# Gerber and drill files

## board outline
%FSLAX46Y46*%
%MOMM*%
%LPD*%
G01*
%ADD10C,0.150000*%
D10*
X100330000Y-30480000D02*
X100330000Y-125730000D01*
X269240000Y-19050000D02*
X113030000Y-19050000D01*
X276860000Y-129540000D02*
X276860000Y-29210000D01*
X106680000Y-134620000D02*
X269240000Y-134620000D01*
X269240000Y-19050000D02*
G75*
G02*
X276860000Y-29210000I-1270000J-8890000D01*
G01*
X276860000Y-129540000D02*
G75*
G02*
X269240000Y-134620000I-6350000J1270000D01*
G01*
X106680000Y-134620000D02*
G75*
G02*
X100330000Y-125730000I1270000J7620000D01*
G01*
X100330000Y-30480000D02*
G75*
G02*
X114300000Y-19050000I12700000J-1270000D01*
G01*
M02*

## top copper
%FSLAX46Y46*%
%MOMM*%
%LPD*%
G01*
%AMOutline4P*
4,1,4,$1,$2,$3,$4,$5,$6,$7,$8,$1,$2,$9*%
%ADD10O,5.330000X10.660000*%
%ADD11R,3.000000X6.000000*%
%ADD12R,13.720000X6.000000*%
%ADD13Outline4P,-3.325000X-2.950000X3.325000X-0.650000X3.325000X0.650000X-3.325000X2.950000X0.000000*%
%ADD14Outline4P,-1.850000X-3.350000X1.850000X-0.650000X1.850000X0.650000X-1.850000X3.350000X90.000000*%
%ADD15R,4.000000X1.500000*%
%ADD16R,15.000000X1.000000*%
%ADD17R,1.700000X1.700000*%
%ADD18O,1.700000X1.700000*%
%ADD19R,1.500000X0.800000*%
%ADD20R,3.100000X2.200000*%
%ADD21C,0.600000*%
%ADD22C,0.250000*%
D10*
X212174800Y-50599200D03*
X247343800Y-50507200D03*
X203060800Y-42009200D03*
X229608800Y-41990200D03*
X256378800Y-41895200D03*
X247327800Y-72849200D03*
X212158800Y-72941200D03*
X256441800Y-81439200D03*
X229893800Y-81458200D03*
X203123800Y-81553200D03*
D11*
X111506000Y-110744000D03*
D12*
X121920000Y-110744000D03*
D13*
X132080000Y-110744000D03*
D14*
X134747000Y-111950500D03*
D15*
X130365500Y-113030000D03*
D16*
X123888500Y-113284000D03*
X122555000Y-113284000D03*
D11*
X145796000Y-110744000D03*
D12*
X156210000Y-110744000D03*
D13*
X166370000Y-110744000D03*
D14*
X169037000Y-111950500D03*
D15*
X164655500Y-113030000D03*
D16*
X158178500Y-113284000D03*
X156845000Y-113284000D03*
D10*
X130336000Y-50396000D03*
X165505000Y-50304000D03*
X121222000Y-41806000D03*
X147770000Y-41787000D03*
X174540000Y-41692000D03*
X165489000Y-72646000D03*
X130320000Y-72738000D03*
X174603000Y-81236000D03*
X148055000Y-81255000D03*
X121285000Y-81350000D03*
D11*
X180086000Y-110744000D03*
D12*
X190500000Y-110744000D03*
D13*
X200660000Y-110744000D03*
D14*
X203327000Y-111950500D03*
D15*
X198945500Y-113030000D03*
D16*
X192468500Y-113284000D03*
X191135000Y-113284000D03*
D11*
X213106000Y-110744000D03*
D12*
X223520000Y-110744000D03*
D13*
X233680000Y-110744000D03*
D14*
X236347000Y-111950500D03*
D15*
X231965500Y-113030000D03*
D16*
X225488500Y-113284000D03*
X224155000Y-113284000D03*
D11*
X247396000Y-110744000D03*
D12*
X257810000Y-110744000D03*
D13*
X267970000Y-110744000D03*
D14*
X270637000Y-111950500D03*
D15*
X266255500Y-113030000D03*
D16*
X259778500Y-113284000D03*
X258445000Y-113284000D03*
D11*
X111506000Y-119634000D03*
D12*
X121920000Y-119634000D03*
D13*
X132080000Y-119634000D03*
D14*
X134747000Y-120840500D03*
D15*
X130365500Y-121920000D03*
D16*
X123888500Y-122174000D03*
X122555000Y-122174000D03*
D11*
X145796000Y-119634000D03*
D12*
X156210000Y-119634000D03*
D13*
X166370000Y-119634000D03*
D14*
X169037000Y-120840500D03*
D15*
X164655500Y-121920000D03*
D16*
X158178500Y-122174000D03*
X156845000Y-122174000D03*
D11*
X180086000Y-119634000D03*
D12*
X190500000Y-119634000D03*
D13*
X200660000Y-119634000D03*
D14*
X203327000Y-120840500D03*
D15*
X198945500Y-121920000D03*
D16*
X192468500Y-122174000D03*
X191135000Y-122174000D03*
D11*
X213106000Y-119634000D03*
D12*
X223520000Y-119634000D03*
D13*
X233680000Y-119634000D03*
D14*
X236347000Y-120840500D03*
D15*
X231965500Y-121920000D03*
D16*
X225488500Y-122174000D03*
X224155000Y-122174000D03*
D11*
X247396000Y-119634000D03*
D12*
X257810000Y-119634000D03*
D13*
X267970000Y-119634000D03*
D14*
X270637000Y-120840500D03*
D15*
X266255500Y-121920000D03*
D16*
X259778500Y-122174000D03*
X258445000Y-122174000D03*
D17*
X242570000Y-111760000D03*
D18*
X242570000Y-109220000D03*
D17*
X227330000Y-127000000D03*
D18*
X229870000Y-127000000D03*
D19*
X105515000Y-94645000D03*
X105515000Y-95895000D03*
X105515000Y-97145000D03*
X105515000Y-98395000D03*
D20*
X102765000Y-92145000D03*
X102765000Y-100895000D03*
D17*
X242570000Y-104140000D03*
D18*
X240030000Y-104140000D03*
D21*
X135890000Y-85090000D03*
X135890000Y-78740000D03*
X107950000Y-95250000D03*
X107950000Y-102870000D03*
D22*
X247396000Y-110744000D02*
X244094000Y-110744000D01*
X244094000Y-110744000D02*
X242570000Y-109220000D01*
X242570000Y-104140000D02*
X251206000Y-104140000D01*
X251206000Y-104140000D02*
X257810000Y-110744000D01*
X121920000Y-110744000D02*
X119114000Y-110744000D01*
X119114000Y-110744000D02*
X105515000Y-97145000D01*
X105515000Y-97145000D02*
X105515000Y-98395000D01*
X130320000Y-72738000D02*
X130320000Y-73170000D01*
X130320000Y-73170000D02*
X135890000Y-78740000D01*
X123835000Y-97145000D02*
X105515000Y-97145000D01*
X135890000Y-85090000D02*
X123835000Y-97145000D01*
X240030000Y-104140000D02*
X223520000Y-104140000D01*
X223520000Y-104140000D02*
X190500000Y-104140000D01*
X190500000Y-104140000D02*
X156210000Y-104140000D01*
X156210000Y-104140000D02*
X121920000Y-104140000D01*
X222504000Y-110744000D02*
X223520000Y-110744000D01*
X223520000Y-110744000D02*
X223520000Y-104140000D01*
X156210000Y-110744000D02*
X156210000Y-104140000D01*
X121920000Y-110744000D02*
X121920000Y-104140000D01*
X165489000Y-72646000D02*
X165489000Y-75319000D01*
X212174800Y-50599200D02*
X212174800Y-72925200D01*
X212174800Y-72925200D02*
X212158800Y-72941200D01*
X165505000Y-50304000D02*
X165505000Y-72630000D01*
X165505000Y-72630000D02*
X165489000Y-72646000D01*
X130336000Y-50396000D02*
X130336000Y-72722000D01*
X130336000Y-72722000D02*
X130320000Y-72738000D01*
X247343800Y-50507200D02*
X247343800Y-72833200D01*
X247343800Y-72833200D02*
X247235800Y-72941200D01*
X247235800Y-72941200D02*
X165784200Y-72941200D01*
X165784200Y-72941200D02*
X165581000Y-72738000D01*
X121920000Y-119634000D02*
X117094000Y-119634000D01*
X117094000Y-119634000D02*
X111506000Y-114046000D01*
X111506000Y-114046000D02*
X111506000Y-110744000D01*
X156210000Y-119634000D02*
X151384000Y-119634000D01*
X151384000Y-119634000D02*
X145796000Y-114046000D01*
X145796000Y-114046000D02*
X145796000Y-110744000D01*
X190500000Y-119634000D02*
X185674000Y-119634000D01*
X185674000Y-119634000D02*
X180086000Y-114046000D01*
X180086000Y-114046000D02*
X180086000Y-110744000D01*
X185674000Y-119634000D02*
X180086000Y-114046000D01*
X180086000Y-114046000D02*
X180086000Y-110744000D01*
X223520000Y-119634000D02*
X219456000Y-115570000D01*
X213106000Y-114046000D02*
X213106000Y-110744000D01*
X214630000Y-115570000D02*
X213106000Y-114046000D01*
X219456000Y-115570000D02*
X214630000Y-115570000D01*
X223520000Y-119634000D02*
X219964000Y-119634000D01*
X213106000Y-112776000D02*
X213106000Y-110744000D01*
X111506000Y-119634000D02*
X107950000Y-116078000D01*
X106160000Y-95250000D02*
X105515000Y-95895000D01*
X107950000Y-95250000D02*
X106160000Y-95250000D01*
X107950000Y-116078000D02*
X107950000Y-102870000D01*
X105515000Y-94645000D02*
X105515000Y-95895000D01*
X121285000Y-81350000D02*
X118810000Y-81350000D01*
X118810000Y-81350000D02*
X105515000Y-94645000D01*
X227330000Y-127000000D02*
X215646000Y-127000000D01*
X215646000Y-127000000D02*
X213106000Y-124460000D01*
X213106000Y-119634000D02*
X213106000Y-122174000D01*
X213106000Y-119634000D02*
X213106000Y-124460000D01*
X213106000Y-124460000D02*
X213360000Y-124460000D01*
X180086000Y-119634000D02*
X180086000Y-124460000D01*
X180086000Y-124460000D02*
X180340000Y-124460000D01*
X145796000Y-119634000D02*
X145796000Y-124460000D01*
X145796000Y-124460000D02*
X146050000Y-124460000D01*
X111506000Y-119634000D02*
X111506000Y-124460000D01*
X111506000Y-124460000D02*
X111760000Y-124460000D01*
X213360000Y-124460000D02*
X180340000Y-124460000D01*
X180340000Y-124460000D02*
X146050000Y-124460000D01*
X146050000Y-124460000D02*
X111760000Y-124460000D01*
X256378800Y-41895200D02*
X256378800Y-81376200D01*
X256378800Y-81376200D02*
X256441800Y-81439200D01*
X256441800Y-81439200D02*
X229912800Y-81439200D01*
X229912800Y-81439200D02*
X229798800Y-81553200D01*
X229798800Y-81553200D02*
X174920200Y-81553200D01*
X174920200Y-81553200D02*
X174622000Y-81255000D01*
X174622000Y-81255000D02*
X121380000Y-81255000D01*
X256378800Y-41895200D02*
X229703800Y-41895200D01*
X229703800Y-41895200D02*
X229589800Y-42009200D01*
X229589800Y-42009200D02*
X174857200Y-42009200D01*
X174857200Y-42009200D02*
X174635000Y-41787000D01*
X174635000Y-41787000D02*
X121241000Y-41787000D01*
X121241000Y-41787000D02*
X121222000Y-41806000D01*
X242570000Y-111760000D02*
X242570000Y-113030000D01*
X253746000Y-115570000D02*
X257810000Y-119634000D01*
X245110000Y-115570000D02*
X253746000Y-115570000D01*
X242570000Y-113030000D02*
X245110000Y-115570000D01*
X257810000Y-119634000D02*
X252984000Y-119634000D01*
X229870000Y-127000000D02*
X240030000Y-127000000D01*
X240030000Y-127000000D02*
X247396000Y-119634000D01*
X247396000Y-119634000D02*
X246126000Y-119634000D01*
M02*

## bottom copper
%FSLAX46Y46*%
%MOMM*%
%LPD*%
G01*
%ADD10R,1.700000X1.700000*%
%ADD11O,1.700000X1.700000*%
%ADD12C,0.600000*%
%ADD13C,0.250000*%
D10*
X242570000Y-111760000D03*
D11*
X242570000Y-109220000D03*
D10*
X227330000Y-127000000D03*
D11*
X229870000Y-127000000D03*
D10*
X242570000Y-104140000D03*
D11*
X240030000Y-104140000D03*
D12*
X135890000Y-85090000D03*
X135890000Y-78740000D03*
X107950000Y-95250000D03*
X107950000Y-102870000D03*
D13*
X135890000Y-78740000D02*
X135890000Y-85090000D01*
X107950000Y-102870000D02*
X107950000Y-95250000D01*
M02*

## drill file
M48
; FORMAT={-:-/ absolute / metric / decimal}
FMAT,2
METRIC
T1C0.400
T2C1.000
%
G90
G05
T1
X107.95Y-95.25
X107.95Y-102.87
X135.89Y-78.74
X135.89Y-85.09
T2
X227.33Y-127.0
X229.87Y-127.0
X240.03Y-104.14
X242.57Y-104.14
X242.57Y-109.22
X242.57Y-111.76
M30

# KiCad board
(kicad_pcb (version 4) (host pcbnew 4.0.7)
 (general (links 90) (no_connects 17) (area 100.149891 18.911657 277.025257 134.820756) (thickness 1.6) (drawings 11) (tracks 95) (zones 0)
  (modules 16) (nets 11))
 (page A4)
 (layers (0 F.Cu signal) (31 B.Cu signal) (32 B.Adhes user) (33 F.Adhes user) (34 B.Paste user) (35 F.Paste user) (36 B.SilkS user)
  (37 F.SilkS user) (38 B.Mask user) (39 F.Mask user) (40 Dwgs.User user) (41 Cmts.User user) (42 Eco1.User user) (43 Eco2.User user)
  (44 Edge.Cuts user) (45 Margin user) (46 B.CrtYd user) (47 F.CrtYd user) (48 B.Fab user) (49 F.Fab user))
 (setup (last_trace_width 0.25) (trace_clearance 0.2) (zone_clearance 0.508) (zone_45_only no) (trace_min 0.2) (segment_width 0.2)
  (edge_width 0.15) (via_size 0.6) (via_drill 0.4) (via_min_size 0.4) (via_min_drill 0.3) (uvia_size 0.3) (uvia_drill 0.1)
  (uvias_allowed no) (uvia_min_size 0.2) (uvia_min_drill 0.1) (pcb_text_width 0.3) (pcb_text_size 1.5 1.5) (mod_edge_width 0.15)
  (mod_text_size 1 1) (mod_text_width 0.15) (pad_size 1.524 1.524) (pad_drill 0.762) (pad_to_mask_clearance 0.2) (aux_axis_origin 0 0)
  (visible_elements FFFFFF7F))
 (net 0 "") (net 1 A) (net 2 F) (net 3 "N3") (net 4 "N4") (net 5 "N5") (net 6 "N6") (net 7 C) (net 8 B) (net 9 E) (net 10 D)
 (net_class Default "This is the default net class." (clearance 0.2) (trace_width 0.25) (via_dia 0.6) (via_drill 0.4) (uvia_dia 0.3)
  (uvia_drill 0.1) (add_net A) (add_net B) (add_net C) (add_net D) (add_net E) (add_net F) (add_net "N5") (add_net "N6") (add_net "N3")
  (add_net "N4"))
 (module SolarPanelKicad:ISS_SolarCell (layer F.Cu) (at 189.7888 101.8032)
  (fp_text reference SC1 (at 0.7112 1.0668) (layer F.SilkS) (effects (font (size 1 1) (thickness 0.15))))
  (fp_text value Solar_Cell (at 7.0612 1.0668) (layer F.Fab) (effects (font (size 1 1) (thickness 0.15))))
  (pad 1 smd oval (at 22.386 -51.204 180) (size 5.33 10.66) (layers F.Cu F.Paste F.Mask) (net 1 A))
  (pad 1 smd oval (at 57.555 -51.296 180) (size 5.33 10.66) (layers F.Cu F.Paste F.Mask) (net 1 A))
  (pad 2 smd oval (at 13.272 -59.794 180) (size 5.33 10.66) (layers F.Cu F.Paste F.Mask) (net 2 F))
  (pad 2 smd oval (at 39.82 -59.813 180) (size 5.33 10.66) (layers F.Cu F.Paste F.Mask) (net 2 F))
  (pad 2 smd oval (at 66.59 -59.908 180) (size 5.33 10.66) (layers F.Cu F.Paste F.Mask) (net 2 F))
  (pad 1 smd oval (at 57.539 -28.954) (size 5.33 10.66) (layers F.Cu F.Paste F.Mask) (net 1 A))
  (pad 1 smd oval (at 22.37 -28.862) (size 5.33 10.66) (layers F.Cu F.Paste F.Mask) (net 1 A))
  (pad 2 smd oval (at 66.653 -20.364) (size 5.33 10.66) (layers F.Cu F.Paste F.Mask) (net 2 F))
  (pad 2 smd oval (at 40.105 -20.345) (size 5.33 10.66) (layers F.Cu F.Paste F.Mask) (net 2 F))
  (pad 2 smd oval (at 13.335 -20.25) (size 5.33 10.66) (layers F.Cu F.Paste F.Mask) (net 2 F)))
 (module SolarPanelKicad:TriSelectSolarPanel (layer F.Cu) (at 113.03 114.3)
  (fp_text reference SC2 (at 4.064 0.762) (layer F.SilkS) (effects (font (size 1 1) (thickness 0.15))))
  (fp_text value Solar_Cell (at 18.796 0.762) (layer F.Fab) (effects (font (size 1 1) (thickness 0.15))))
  (pad 2 smd rect (at -1.524 -3.556) (size 3 6) (layers F.Cu F.Paste F.Mask) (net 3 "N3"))
  (pad 1 smd rect (at 8.89 -3.556) (size 13.72 6) (layers F.Cu F.Paste F.Mask) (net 1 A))
  (pad 1 smd trapezoid (at 19.05 -3.556) (size 6.65 3.6) (rect_delta 2.3 0) (layers F.Cu F.Paste F.Mask) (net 1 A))
  (pad 1 smd trapezoid (at 21.717 -2.3495 90) (size 3.7 4) (rect_delta 2.7 0) (layers F.Cu F.Paste F.Mask) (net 1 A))
  (pad 1 smd rect (at 17.3355 -1.27) (size 4 1.5) (layers F.Cu F.Paste F.Mask) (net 1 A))
  (pad 1 smd rect (at 10.8585 -1.016) (size 15 1) (layers F.Cu F.Paste F.Mask) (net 1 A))
  (pad 1 smd rect (at 9.525 -1.016) (size 15 1) (layers F.Cu F.Paste F.Mask) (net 1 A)))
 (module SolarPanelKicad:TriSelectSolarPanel (layer F.Cu) (at 147.32 114.3)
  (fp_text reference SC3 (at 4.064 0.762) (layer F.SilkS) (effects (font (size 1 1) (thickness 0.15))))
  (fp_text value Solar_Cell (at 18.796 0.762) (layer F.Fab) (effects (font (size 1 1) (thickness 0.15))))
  (pad 2 smd rect (at -1.524 -3.556) (size 3 6) (layers F.Cu F.Paste F.Mask) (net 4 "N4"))
  (pad 1 smd rect (at 8.89 -3.556) (size 13.72 6) (layers F.Cu F.Paste F.Mask) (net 1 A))
  (pad 1 smd trapezoid (at 19.05 -3.556) (size 6.65 3.6) (rect_delta 2.3 0) (layers F.Cu F.Paste F.Mask) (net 1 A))
  (pad 1 smd trapezoid (at 21.717 -2.3495 90) (size 3.7 4) (rect_delta 2.7 0) (layers F.Cu F.Paste F.Mask) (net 1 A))
  (pad 1 smd rect (at 17.3355 -1.27) (size 4 1.5) (layers F.Cu F.Paste F.Mask) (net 1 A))
  (pad 1 smd rect (at 10.8585 -1.016) (size 15 1) (layers F.Cu F.Paste F.Mask) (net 1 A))
  (pad 1 smd rect (at 9.525 -1.016) (size 15 1) (layers F.Cu F.Paste F.Mask) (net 1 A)))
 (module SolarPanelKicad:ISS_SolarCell (layer F.Cu) (at 107.95 101.6)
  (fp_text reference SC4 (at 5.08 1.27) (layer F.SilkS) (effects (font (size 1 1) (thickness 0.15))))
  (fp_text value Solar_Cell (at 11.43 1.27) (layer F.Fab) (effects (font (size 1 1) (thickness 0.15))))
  (pad 1 smd oval (at 22.386 -51.204 180) (size 5.33 10.66) (layers F.Cu F.Paste F.Mask) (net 1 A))
  (pad 1 smd oval (at 57.555 -51.296 180) (size 5.33 10.66) (layers F.Cu F.Paste F.Mask) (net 1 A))
  (pad 2 smd oval (at 13.272 -59.794 180) (size 5.33 10.66) (layers F.Cu F.Paste F.Mask) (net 2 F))
  (pad 2 smd oval (at 39.82 -59.813 180) (size 5.33 10.66) (layers F.Cu F.Paste F.Mask) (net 2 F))
  (pad 2 smd oval (at 66.59 -59.908 180) (size 5.33 10.66) (layers F.Cu F.Paste F.Mask) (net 2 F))
  (pad 1 smd oval (at 57.539 -28.954) (size 5.33 10.66) (layers F.Cu F.Paste F.Mask) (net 1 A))
  (pad 1 smd oval (at 22.37 -28.862) (size 5.33 10.66) (layers F.Cu F.Paste F.Mask) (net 1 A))
  (pad 2 smd oval (at 66.653 -20.364) (size 5.33 10.66) (layers F.Cu F.Paste F.Mask) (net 2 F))
  (pad 2 smd oval (at 40.105 -20.345) (size 5.33 10.66) (layers F.Cu F.Paste F.Mask) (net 2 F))
  (pad 2 smd oval (at 13.335 -20.25) (size 5.33 10.66) (layers F.Cu F.Paste F.Mask) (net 2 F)))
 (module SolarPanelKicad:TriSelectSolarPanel (layer F.Cu) (at 181.61 114.3)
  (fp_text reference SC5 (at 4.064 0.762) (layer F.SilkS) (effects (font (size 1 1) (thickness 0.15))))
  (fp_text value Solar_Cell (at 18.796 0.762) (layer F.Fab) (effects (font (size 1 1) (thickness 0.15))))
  (pad 2 smd rect (at -1.524 -3.556) (size 3 6) (layers F.Cu F.Paste F.Mask) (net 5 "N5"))
  (pad 1 smd rect (at 8.89 -3.556) (size 13.72 6) (layers F.Cu F.Paste F.Mask) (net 1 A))
  (pad 1 smd trapezoid (at 19.05 -3.556) (size 6.65 3.6) (rect_delta 2.3 0) (layers F.Cu F.Paste F.Mask) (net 1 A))
  (pad 1 smd trapezoid (at 21.717 -2.3495 90) (size 3.7 4) (rect_delta 2.7 0) (layers F.Cu F.Paste F.Mask) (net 1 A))
  (pad 1 smd rect (at 17.3355 -1.27) (size 4 1.5) (layers F.Cu F.Paste F.Mask) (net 1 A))
  (pad 1 smd rect (at 10.8585 -1.016) (size 15 1) (layers F.Cu F.Paste F.Mask) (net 1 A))
  (pad 1 smd rect (at 9.525 -1.016) (size 15 1) (layers F.Cu F.Paste F.Mask) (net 1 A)))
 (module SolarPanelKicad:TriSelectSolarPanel (layer F.Cu) (at 214.63 114.3)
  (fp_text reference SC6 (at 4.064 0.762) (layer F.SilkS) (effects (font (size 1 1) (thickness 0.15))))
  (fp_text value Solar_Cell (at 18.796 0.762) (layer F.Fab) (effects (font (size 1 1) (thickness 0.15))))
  (pad 2 smd rect (at -1.524 -3.556) (size 3 6) (layers F.Cu F.Paste F.Mask) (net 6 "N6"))
  (pad 1 smd rect (at 8.89 -3.556) (size 13.72 6) (layers F.Cu F.Paste F.Mask) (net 1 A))
  (pad 1 smd trapezoid (at 19.05 -3.556) (size 6.65 3.6) (rect_delta 2.3 0) (layers F.Cu F.Paste F.Mask) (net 1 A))
  (pad 1 smd trapezoid (at 21.717 -2.3495 90) (size 3.7 4) (rect_delta 2.7 0) (layers F.Cu F.Paste F.Mask) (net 1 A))
  (pad 1 smd rect (at 17.3355 -1.27) (size 4 1.5) (layers F.Cu F.Paste F.Mask) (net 1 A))
  (pad 1 smd rect (at 10.8585 -1.016) (size 15 1) (layers F.Cu F.Paste F.Mask) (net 1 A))
  (pad 1 smd rect (at 9.525 -1.016) (size 15 1) (layers F.Cu F.Paste F.Mask) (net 1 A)))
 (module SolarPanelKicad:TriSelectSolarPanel (layer F.Cu) (at 248.92 114.3)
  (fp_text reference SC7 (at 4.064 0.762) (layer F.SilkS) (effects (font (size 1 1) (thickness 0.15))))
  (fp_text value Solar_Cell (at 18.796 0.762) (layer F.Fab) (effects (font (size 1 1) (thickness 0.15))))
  (pad 2 smd rect (at -1.524 -3.556) (size 3 6) (layers F.Cu F.Paste F.Mask) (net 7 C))
  (pad 1 smd rect (at 8.89 -3.556) (size 13.72 6) (layers F.Cu F.Paste F.Mask) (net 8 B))
  (pad 1 smd trapezoid (at 19.05 -3.556) (size 6.65 3.6) (rect_delta 2.3 0) (layers F.Cu F.Paste F.Mask) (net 8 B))
  (pad 1 smd trapezoid (at 21.717 -2.3495 90) (size 3.7 4) (rect_delta 2.7 0) (layers F.Cu F.Paste F.Mask) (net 8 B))
  (pad 1 smd rect (at 17.3355 -1.27) (size 4 1.5) (layers F.Cu F.Paste F.Mask) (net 8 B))
  (pad 1 smd rect (at 10.8585 -1.016) (size 15 1) (layers F.Cu F.Paste F.Mask) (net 8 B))
  (pad 1 smd rect (at 9.525 -1.016) (size 15 1) (layers F.Cu F.Paste F.Mask) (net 8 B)))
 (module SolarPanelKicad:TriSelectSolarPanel (layer F.Cu) (at 113.03 123.19)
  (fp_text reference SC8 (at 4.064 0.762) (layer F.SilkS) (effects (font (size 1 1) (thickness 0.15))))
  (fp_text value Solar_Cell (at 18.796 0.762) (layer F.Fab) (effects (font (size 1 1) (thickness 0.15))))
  (pad 2 smd rect (at -1.524 -3.556) (size 3 6) (layers F.Cu F.Paste F.Mask) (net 2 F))
  (pad 1 smd rect (at 8.89 -3.556) (size 13.72 6) (layers F.Cu F.Paste F.Mask) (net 3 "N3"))
  (pad 1 smd trapezoid (at 19.05 -3.556) (size 6.65 3.6) (rect_delta 2.3 0) (layers F.Cu F.Paste F.Mask) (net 3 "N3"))
  (pad 1 smd trapezoid (at 21.717 -2.3495 90) (size 3.7 4) (rect_delta 2.7 0) (layers F.Cu F.Paste F.Mask) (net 3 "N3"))
  (pad 1 smd rect (at 17.3355 -1.27) (size 4 1.5) (layers F.Cu F.Paste F.Mask) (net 3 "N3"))
  (pad 1 smd rect (at 10.8585 -1.016) (size 15 1) (layers F.Cu F.Paste F.Mask) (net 3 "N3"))
  (pad 1 smd rect (at 9.525 -1.016) (size 15 1) (layers F.Cu F.Paste F.Mask) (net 3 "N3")))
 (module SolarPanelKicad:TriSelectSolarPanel (layer F.Cu) (at 147.32 123.19)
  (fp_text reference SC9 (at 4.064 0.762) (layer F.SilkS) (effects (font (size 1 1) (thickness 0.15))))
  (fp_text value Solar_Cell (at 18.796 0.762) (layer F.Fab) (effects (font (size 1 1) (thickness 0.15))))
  (pad 2 smd rect (at -1.524 -3.556) (size 3 6) (layers F.Cu F.Paste F.Mask) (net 2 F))
  (pad 1 smd rect (at 8.89 -3.556) (size 13.72 6) (layers F.Cu F.Paste F.Mask) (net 4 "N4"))
  (pad 1 smd trapezoid (at 19.05 -3.556) (size 6.65 3.6) (rect_delta 2.3 0) (layers F.Cu F.Paste F.Mask) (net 4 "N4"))
  (pad 1 smd trapezoid (at 21.717 -2.3495 90) (size 3.7 4) (rect_delta 2.7 0) (layers F.Cu F.Paste F.Mask) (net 4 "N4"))
  (pad 1 smd rect (at 17.3355 -1.27) (size 4 1.5) (layers F.Cu F.Paste F.Mask) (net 4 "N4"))
  (pad 1 smd rect (at 10.8585 -1.016) (size 15 1) (layers F.Cu F.Paste F.Mask) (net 4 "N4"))
  (pad 1 smd rect (at 9.525 -1.016) (size 15 1) (layers F.Cu F.Paste F.Mask) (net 4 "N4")))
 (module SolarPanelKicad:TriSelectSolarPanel (layer F.Cu) (at 181.61 123.19)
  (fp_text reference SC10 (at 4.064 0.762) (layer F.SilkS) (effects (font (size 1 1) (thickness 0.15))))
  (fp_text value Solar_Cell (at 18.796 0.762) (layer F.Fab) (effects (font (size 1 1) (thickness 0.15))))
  (pad 2 smd rect (at -1.524 -3.556) (size 3 6) (layers F.Cu F.Paste F.Mask) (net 2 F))
  (pad 1 smd rect (at 8.89 -3.556) (size 13.72 6) (layers F.Cu F.Paste F.Mask) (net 5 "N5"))
  (pad 1 smd trapezoid (at 19.05 -3.556) (size 6.65 3.6) (rect_delta 2.3 0) (layers F.Cu F.Paste F.Mask) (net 5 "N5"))
  (pad 1 smd trapezoid (at 21.717 -2.3495 90) (size 3.7 4) (rect_delta 2.7 0) (layers F.Cu F.Paste F.Mask) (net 5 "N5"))
  (pad 1 smd rect (at 17.3355 -1.27) (size 4 1.5) (layers F.Cu F.Paste F.Mask) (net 5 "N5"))
  (pad 1 smd rect (at 10.8585 -1.016) (size 15 1) (layers F.Cu F.Paste F.Mask) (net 5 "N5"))
  (pad 1 smd rect (at 9.525 -1.016) (size 15 1) (layers F.Cu F.Paste F.Mask) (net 5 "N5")))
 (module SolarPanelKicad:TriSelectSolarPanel (layer F.Cu) (at 214.63 123.19)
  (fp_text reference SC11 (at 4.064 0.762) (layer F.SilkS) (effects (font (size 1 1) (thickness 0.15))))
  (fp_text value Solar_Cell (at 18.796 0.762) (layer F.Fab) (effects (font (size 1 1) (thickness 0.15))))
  (pad 2 smd rect (at -1.524 -3.556) (size 3 6) (layers F.Cu F.Paste F.Mask) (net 2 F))
  (pad 1 smd rect (at 8.89 -3.556) (size 13.72 6) (layers F.Cu F.Paste F.Mask) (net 6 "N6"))
  (pad 1 smd trapezoid (at 19.05 -3.556) (size 6.65 3.6) (rect_delta 2.3 0) (layers F.Cu F.Paste F.Mask) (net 6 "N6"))
  (pad 1 smd trapezoid (at 21.717 -2.3495 90) (size 3.7 4) (rect_delta 2.7 0) (layers F.Cu F.Paste F.Mask) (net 6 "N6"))
  (pad 1 smd rect (at 17.3355 -1.27) (size 4 1.5) (layers F.Cu F.Paste F.Mask) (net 6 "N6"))
  (pad 1 smd rect (at 10.8585 -1.016) (size 15 1) (layers F.Cu F.Paste F.Mask) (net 6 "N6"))
  (pad 1 smd rect (at 9.525 -1.016) (size 15 1) (layers F.Cu F.Paste F.Mask) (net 6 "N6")))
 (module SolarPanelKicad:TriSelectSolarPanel (layer F.Cu) (at 248.92 123.19)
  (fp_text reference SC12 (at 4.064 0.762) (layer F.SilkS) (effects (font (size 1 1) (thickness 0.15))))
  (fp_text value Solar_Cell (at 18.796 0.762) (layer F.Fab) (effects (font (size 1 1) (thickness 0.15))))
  (pad 2 smd rect (at -1.524 -3.556) (size 3 6) (layers F.Cu F.Paste F.Mask) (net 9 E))
  (pad 1 smd rect (at 8.89 -3.556) (size 13.72 6) (layers F.Cu F.Paste F.Mask) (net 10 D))
  (pad 1 smd trapezoid (at 19.05 -3.556) (size 6.65 3.6) (rect_delta 2.3 0) (layers F.Cu F.Paste F.Mask) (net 10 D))
  (pad 1 smd trapezoid (at 21.717 -2.3495 90) (size 3.7 4) (rect_delta 2.7 0) (layers F.Cu F.Paste F.Mask) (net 10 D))
  (pad 1 smd rect (at 17.3355 -1.27) (size 4 1.5) (layers F.Cu F.Paste F.Mask) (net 10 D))
  (pad 1 smd rect (at 10.8585 -1.016) (size 15 1) (layers F.Cu F.Paste F.Mask) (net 10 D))
  (pad 1 smd rect (at 9.525 -1.016) (size 15 1) (layers F.Cu F.Paste F.Mask) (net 10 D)))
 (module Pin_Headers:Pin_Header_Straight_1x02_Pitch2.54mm (layer F.Cu) (at 242.57 111.76 180)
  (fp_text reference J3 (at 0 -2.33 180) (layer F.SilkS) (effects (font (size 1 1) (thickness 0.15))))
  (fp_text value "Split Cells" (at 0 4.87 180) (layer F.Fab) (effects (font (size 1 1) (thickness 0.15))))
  (pad 1 thru_hole rect (at 0 0 180) (size 1.7 1.7) (drill 1) (layers *.Cu *.Mask) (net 10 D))
  (pad 2 thru_hole oval (at 0 2.54 180) (size 1.7 1.7) (drill 1) (layers *.Cu *.Mask) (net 7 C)))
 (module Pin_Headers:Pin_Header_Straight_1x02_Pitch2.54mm (layer F.Cu) (at 227.33 127 90)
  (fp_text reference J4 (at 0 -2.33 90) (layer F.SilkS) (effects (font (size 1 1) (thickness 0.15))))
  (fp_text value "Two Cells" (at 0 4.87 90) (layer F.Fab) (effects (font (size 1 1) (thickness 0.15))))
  (pad 1 thru_hole rect (at 0 0 90) (size 1.7 1.7) (drill 1) (layers *.Cu *.Mask) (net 2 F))
  (pad 2 thru_hole oval (at 0 2.54 90) (size 1.7 1.7) (drill 1) (layers *.Cu *.Mask) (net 9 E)))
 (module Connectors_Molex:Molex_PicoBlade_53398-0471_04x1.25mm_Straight (layer F.Cu) (at 104.14 96.52 270)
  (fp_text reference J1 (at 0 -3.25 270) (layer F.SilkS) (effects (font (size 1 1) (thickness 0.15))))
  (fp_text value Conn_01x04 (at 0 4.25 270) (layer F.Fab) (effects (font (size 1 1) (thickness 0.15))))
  (pad 1 smd rect (at -1.875 -1.375 270) (size 0.8 1.5) (layers F.Cu F.Paste F.Mask) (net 2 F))
  (pad 2 smd rect (at -0.625 -1.375 270) (size 0.8 1.5) (layers F.Cu F.Paste F.Mask) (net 2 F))
  (pad 3 smd rect (at 0.625 -1.375 270) (size 0.8 1.5) (layers F.Cu F.Paste F.Mask) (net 1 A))
  (pad 4 smd rect (at 1.875 -1.375 270) (size 0.8 1.5) (layers F.Cu F.Paste F.Mask) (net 1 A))
  (pad "" smd rect (at -4.375 1.375 270) (size 2.2 3.1) (layers F.Cu F.Paste F.Mask))
  (pad "" smd rect (at 4.375 1.375 270) (size 2.2 3.1) (layers F.Cu F.Paste F.Mask)))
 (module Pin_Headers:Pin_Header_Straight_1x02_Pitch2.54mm (layer F.Cu) (at 242.57 104.14 270)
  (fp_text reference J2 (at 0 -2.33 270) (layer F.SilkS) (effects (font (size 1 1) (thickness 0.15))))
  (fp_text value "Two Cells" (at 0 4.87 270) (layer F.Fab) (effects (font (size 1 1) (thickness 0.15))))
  (pad 1 thru_hole rect (at 0 0 270) (size 1.7 1.7) (drill 1) (layers *.Cu *.Mask) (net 8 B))
  (pad 2 thru_hole oval (at 0 2.54 270) (size 1.7 1.7) (drill 1) (layers *.Cu *.Mask) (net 1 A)))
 (gr_line (start 100.33 30.48) (end 100.33 125.73) (angle 90) (layer Edge.Cuts) (width 0.15))
 (gr_line (start 269.24 19.05) (end 113.03 19.05) (angle 90) (layer Edge.Cuts) (width 0.15))
 (gr_line (start 276.86 129.54) (end 276.86 29.21) (angle 90) (layer Edge.Cuts) (width 0.15))
 (gr_line (start 106.68 134.62) (end 269.24 134.62) (angle 90) (layer Edge.Cuts) (width 0.15))
 (gr_arc (start 267.97 27.94) (end 269.24 19.05) (angle 90) (layer Edge.Cuts) (width 0.15))
 (gr_arc (start 270.51 128.27) (end 276.86 129.54) (angle 90) (layer Edge.Cuts) (width 0.15))
 (gr_arc (start 107.95 127) (end 106.68 134.62) (angle 90) (layer Edge.Cuts) (width 0.15))
 (gr_arc (start 113.03 31.75) (end 100.33 30.48) (angle 90) (layer Edge.Cuts) (width 0.15))
 (segment (start 247.396 110.744) (end 244.094 110.744) (width 0.25) (layer F.Cu) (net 7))
 (segment (start 244.094 110.744) (end 242.57 109.22) (width 0.25) (layer F.Cu) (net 7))
 (segment (start 242.57 104.14) (end 251.206 104.14) (width 0.25) (layer F.Cu) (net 8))
 (segment (start 251.206 104.14) (end 257.81 110.744) (width 0.25) (layer F.Cu) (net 8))
 (segment (start 121.92 110.744) (end 119.114 110.744) (width 0.25) (layer F.Cu) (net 1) (status C00000))
 (segment (start 119.114 110.744) (end 105.515 97.145) (width 0.25) (layer F.Cu) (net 1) (status C00000))
 (segment (start 105.515 97.145) (end 105.515 98.395) (width 0.25) (layer F.Cu) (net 1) (status C00000))
 (segment (start 130.32 72.738) (end 130.32 73.17) (width 0.25) (layer F.Cu) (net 1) (status C00000))
 (segment (start 130.32 73.17) (end 135.89 78.74) (width 0.25) (layer F.Cu) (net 1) (status 400000))
 (segment (start 123.835 97.145) (end 105.515 97.145) (width 0.25) (layer F.Cu) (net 1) (status 800000))
 (segment (start 135.89 85.09) (end 123.835 97.145) (width 0.25) (layer F.Cu) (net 1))
 (via (at 135.89 85.09) (size 0.6) (drill 0.4) (layers F.Cu B.Cu) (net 1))
 (segment (start 135.89 78.74) (end 135.89 85.09) (width 0.25) (layer B.Cu) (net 1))
 (via (at 135.89 78.74) (size 0.6) (drill 0.4) (layers F.Cu B.Cu) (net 1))
 (segment (start 240.03 104.14) (end 223.52 104.14) (width 0.25) (layer F.Cu) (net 1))
 (segment (start 223.52 104.14) (end 190.5 104.14) (width 0.25) (layer F.Cu) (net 1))
 (segment (start 190.5 104.14) (end 156.21 104.14) (width 0.25) (layer F.Cu) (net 1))
 (segment (start 156.21 104.14) (end 121.92 104.14) (width 0.25) (layer F.Cu) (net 1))
 (segment (start 222.504 110.744) (end 223.52 110.744) (width 0.25) (layer F.Cu) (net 1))
 (segment (start 223.52 110.744) (end 223.52 104.14) (width 0.25) (layer F.Cu) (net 1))
 (segment (start 156.21 110.744) (end 156.21 104.14) (width 0.25) (layer F.Cu) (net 1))
 (segment (start 121.92 110.744) (end 121.92 104.14) (width 0.25) (layer F.Cu) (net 1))
 (segment (start 165.489 72.646) (end 165.489 75.319) (width 0.25) (layer F.Cu) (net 1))
 (segment (start 212.1748 50.5992) (end 212.1748 72.9252) (width 0.25) (layer F.Cu) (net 1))
 (segment (start 212.1748 72.9252) (end 212.1588 72.9412) (width 0.25) (layer F.Cu) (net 1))
 (segment (start 165.505 50.304) (end 165.505 72.63) (width 0.25) (layer F.Cu) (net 1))
 (segment (start 165.505 72.63) (end 165.489 72.646) (width 0.25) (layer F.Cu) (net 1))
 (segment (start 130.336 50.396) (end 130.336 72.722) (width 0.25) (layer F.Cu) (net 1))
 (segment (start 130.336 72.722) (end 130.32 72.738) (width 0.25) (layer F.Cu) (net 1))
 (segment (start 247.3438 50.5072) (end 247.3438 72.8332) (width 0.25) (layer F.Cu) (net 1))
 (segment (start 247.3438 72.8332) (end 247.2358 72.9412) (width 0.25) (layer F.Cu) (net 1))
 (segment (start 247.2358 72.9412) (end 165.7842 72.9412) (width 0.25) (layer F.Cu) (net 1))
 (segment (start 165.7842 72.9412) (end 165.581 72.738) (width 0.25) (layer F.Cu) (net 1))
 (segment (start 121.92 119.634) (end 117.094 119.634) (width 0.25) (layer F.Cu) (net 3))
 (segment (start 117.094 119.634) (end 111.506 114.046) (width 0.25) (layer F.Cu) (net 3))
 (segment (start 111.506 114.046) (end 111.506 110.744) (width 0.25) (layer F.Cu) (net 3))
 (segment (start 156.21 119.634) (end 151.384 119.634) (width 0.25) (layer F.Cu) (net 4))
 (segment (start 151.384 119.634) (end 145.796 114.046) (width 0.25) (layer F.Cu) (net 4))
 (segment (start 145.796 114.046) (end 145.796 110.744) (width 0.25) (layer F.Cu) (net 4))
 (segment (start 190.5 119.634) (end 185.674 119.634) (width 0.25) (layer F.Cu) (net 5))
 (segment (start 185.674 119.634) (end 180.086 114.046) (width 0.25) (layer F.Cu) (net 5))
 (segment (start 180.086 114.046) (end 180.086 110.744) (width 0.25) (layer F.Cu) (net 5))
 (segment (start 185.674 119.634) (end 180.086 114.046) (width 0.25) (layer F.Cu) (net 5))
 (segment (start 180.086 114.046) (end 180.086 110.744) (width 0.25) (layer F.Cu) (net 5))
 (segment (start 223.52 119.634) (end 219.456 115.57) (width 0.25) (layer F.Cu) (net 6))
 (segment (start 213.106 114.046) (end 213.106 110.744) (width 0.25) (layer F.Cu) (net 6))
 (segment (start 214.63 115.57) (end 213.106 114.046) (width 0.25) (layer F.Cu) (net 6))
 (segment (start 219.456 115.57) (end 214.63 115.57) (width 0.25) (layer F.Cu) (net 6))
 (segment (start 223.52 119.634) (end 219.964 119.634) (width 0.25) (layer F.Cu) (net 6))
 (segment (start 213.106 112.776) (end 213.106 110.744) (width 0.25) (layer F.Cu) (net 6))
 (segment (start 111.506 119.634) (end 107.95 116.078) (width 0.25) (layer F.Cu) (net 2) (status 400000))
 (segment (start 106.16 95.25) (end 105.515 95.895) (width 0.25) (layer F.Cu) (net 2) (status 800000))
 (segment (start 107.95 95.25) (end 106.16 95.25) (width 0.25) (layer F.Cu) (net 2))
 (via (at 107.95 95.25) (size 0.6) (drill 0.4) (layers F.Cu B.Cu) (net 2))
 (segment (start 107.95 102.87) (end 107.95 95.25) (width 0.25) (layer B.Cu) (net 2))
 (via (at 107.95 102.87) (size 0.6) (drill 0.4) (layers F.Cu B.Cu) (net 2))
 (segment (start 107.95 116.078) (end 107.95 102.87) (width 0.25) (layer F.Cu) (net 2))
 (segment (start 105.515 94.645) (end 105.515 95.895) (width 0.25) (layer F.Cu) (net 2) (status C00000))
 (segment (start 121.285 81.35) (end 118.81 81.35) (width 0.25) (layer F.Cu) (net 2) (status C00000))
 (segment (start 118.81 81.35) (end 105.515 94.645) (width 0.25) (layer F.Cu) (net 2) (status C00000))
 (segment (start 227.33 127) (end 215.646 127) (width 0.25) (layer F.Cu) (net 2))
 (segment (start 215.646 127) (end 213.106 124.46) (width 0.25) (layer F.Cu) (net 2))
 (segment (start 213.106 119.634) (end 213.106 122.174) (width 0.25) (layer F.Cu) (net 2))
 (segment (start 213.106 119.634) (end 213.106 124.46) (width 0.25) (layer F.Cu) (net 2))
 (segment (start 213.106 124.46) (end 213.36 124.46) (width 0.25) (layer F.Cu) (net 2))
 (segment (start 180.086 119.634) (end 180.086 124.46) (width 0.25) (layer F.Cu) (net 2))
 (segment (start 180.086 124.46) (end 180.34 124.46) (width 0.25) (layer F.Cu) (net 2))
 (segment (start 145.796 119.634) (end 145.796 124.46) (width 0.25) (layer F.Cu) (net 2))
 (segment (start 145.796 124.46) (end 146.05 124.46) (width 0.25) (layer F.Cu) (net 2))
 (segment (start 111.506 119.634) (end 111.506 124.46) (width 0.25) (layer F.Cu) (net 2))
 (segment (start 111.506 124.46) (end 111.76 124.46) (width 0.25) (layer F.Cu) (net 2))
 (segment (start 213.36 124.46) (end 180.34 124.46) (width 0.25) (layer F.Cu) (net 2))
 (segment (start 180.34 124.46) (end 146.05 124.46) (width 0.25) (layer F.Cu) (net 2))
 (segment (start 146.05 124.46) (end 111.76 124.46) (width 0.25) (layer F.Cu) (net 2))
 (segment (start 256.3788 41.8952) (end 256.3788 81.3762) (width 0.25) (layer F.Cu) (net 2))
 (segment (start 256.3788 81.3762) (end 256.4418 81.4392) (width 0.25) (layer F.Cu) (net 2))
 (segment (start 256.4418 81.4392) (end 229.9128 81.4392) (width 0.25) (layer F.Cu) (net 2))
 (segment (start 229.9128 81.4392) (end 229.7988 81.5532) (width 0.25) (layer F.Cu) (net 2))
 (segment (start 229.7988 81.5532) (end 174.9202 81.5532) (width 0.25) (layer F.Cu) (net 2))
 (segment (start 174.9202 81.5532) (end 174.622 81.255) (width 0.25) (layer F.Cu) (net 2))
 (segment (start 174.622 81.255) (end 121.38 81.255) (width 0.25) (layer F.Cu) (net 2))
 (segment (start 256.3788 41.8952) (end 229.7038 41.8952) (width 0.25) (layer F.Cu) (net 2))
 (segment (start 229.7038 41.8952) (end 229.5898 42.0092) (width 0.25) (layer F.Cu) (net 2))
 (segment (start 229.5898 42.0092) (end 174.8572 42.0092) (width 0.25) (layer F.Cu) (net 2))
 (segment (start 174.8572 42.0092) (end 174.635 41.787) (width 0.25) (layer F.Cu) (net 2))
 (segment (start 174.635 41.787) (end 121.241 41.787) (width 0.25) (layer F.Cu) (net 2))
 (segment (start 121.241 41.787) (end 121.222 41.806) (width 0.25) (layer F.Cu) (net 2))
 (segment (start 242.57 111.76) (end 242.57 113.03) (width 0.25) (layer F.Cu) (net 10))
 (segment (start 253.746 115.57) (end 257.81 119.634) (width 0.25) (layer F.Cu) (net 10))
 (segment (start 245.11 115.57) (end 253.746 115.57) (width 0.25) (layer F.Cu) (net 10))
 (segment (start 242.57 113.03) (end 245.11 115.57) (width 0.25) (layer F.Cu) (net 10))
 (segment (start 257.81 119.634) (end 252.984 119.634) (width 0.25) (layer F.Cu) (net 10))
 (segment (start 229.87 127) (end 240.03 127) (width 0.25) (layer F.Cu) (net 9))
 (segment (start 240.03 127) (end 247.396 119.634) (width 0.25) (layer F.Cu) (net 9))
 (segment (start 247.396 119.634) (end 246.126 119.634) (width 0.25) (layer F.Cu) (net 9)))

